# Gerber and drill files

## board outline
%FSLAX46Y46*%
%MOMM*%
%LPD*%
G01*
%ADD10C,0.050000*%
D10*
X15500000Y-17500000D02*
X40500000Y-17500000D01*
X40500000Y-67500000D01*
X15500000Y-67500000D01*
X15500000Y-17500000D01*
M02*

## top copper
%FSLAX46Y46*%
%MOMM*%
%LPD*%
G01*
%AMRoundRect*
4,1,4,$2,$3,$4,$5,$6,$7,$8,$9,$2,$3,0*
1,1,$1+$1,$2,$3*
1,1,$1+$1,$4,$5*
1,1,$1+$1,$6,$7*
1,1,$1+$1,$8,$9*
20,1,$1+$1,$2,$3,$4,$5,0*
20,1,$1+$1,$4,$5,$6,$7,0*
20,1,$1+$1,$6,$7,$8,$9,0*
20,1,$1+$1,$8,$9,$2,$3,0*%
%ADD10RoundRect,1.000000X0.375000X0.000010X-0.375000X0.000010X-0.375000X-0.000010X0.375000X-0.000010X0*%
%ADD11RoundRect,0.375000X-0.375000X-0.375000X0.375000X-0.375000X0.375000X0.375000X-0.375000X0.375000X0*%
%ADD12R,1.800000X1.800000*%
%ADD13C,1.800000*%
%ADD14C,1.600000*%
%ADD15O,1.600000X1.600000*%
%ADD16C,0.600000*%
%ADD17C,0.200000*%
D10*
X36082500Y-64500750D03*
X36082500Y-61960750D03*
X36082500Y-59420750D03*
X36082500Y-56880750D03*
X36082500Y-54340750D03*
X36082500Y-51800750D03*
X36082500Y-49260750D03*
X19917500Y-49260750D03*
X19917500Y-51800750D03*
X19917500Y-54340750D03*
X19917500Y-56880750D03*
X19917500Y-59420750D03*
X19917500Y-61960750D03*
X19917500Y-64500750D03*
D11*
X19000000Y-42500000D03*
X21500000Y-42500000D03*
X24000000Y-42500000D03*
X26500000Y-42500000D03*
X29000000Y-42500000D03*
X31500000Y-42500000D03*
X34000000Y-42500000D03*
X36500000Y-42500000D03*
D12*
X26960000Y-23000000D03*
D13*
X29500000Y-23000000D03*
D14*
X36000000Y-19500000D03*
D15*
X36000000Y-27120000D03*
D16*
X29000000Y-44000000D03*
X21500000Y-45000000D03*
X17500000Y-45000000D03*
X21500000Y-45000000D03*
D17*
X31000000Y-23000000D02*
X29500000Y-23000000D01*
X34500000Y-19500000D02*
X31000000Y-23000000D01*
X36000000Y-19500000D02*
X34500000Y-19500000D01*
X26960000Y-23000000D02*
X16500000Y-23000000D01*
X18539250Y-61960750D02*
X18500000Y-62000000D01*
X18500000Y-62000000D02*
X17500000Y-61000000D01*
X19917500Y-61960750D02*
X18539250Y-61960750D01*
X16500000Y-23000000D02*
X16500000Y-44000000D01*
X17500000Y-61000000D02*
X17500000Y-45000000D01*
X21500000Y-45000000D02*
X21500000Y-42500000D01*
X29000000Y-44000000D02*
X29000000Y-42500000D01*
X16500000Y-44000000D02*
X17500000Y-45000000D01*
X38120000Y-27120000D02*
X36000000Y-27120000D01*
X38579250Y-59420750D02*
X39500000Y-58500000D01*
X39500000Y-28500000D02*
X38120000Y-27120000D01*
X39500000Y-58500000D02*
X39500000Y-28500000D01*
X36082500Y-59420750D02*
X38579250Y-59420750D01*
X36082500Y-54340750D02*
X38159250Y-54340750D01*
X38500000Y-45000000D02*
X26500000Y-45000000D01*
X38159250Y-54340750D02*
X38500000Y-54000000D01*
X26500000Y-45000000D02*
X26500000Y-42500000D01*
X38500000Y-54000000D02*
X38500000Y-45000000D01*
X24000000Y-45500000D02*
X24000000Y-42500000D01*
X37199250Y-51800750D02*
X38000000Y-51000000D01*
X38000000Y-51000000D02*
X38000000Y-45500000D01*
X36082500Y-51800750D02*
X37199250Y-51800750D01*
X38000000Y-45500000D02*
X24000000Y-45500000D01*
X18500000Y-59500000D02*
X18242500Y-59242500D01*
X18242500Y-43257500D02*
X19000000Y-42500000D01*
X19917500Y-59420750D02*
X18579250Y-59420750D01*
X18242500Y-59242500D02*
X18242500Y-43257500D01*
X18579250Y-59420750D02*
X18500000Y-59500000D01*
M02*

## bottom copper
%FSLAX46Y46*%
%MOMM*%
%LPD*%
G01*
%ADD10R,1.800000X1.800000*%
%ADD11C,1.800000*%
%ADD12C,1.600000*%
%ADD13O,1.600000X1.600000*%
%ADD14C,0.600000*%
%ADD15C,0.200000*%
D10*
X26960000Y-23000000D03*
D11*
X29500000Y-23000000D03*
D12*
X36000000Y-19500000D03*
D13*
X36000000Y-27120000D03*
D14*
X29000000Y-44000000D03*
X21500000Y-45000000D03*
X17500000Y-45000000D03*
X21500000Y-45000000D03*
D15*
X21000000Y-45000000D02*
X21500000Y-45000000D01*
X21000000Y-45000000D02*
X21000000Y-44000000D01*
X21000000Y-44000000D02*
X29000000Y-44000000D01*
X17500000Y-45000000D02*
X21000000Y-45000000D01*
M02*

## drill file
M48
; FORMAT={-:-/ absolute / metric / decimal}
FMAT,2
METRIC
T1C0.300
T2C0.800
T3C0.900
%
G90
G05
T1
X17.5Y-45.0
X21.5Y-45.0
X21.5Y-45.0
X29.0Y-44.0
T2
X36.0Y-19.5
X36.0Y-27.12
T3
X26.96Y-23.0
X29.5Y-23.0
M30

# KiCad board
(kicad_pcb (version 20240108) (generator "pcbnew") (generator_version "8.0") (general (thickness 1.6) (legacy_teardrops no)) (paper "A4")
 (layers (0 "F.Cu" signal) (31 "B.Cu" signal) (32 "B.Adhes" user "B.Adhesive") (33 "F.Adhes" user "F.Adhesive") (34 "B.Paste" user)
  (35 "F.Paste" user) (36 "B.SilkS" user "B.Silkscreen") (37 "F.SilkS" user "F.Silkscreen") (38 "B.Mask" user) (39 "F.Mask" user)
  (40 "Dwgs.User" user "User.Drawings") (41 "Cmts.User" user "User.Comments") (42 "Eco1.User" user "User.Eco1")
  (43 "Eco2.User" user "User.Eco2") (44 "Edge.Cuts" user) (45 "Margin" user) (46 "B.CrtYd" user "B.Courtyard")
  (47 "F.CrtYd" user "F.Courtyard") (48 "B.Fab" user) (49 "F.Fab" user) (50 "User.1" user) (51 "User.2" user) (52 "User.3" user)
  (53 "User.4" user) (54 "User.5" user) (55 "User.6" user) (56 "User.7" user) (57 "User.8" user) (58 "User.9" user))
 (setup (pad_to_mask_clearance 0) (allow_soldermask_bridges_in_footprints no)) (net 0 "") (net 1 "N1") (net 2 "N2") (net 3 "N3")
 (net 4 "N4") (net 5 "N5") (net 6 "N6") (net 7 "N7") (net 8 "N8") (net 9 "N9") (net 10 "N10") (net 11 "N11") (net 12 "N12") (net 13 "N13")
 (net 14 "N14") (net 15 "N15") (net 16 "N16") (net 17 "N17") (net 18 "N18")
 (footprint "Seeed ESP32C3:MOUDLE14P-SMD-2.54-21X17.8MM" (layer "F.Cu") (at 36.9175 46.38075 180)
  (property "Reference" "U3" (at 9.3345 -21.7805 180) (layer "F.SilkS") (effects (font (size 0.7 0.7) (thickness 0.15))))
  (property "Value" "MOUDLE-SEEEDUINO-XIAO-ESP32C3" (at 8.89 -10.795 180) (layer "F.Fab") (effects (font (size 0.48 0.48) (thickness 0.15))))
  (pad "1" smd roundrect (at 0.835 -18.12 180) (size 2.75 2) (layers "F.Cu" "F.Paste" "F.Mask") (roundrect_rratio 0.5) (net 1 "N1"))
  (pad "2" smd roundrect (at 0.835 -15.58 180) (size 2.75 2) (layers "F.Cu" "F.Paste" "F.Mask") (roundrect_rratio 0.5) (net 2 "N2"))
  (pad "3" smd roundrect (at 0.835 -13.04 180) (size 2.75 2) (layers "F.Cu" "F.Paste" "F.Mask") (roundrect_rratio 0.5) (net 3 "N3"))
  (pad "4" smd roundrect (at 0.835 -10.5 180) (size 2.75 2) (layers "F.Cu" "F.Paste" "F.Mask") (roundrect_rratio 0.5) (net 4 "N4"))
  (pad "5" smd roundrect (at 0.835 -7.96 180) (size 2.75 2) (layers "F.Cu" "F.Paste" "F.Mask") (roundrect_rratio 0.5) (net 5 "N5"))
  (pad "6" smd roundrect (at 0.835 -5.42 180) (size 2.75 2) (layers "F.Cu" "F.Paste" "F.Mask") (roundrect_rratio 0.5) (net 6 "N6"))
  (pad "7" smd roundrect (at 0.835 -2.88 180) (size 2.75 2) (layers "F.Cu" "F.Paste" "F.Mask") (roundrect_rratio 0.5) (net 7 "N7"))
  (pad "8" smd roundrect (at 17 -2.88 180) (size 2.75 2) (layers "F.Cu" "F.Paste" "F.Mask") (roundrect_rratio 0.5) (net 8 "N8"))
  (pad "9" smd roundrect (at 17 -5.42 180) (size 2.75 2) (layers "F.Cu" "F.Paste" "F.Mask") (roundrect_rratio 0.5) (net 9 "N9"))
  (pad "10" smd roundrect (at 17 -7.96 180) (size 2.75 2) (layers "F.Cu" "F.Paste" "F.Mask") (roundrect_rratio 0.5) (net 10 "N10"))
  (pad "11" smd roundrect (at 17 -10.5 180) (size 2.75 2) (layers "F.Cu" "F.Paste" "F.Mask") (roundrect_rratio 0.5) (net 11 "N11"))
  (pad "12" smd roundrect (at 17 -13.04 180) (size 2.75 2) (layers "F.Cu" "F.Paste" "F.Mask") (roundrect_rratio 0.5) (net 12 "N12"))
  (pad "13" smd roundrect (at 17 -15.58 180) (size 2.75 2) (layers "F.Cu" "F.Paste" "F.Mask") (roundrect_rratio 0.5) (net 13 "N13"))
  (pad "14" smd roundrect (at 17 -18.12 180) (size 2.75 2) (layers "F.Cu" "F.Paste" "F.Mask") (roundrect_rratio 0.5) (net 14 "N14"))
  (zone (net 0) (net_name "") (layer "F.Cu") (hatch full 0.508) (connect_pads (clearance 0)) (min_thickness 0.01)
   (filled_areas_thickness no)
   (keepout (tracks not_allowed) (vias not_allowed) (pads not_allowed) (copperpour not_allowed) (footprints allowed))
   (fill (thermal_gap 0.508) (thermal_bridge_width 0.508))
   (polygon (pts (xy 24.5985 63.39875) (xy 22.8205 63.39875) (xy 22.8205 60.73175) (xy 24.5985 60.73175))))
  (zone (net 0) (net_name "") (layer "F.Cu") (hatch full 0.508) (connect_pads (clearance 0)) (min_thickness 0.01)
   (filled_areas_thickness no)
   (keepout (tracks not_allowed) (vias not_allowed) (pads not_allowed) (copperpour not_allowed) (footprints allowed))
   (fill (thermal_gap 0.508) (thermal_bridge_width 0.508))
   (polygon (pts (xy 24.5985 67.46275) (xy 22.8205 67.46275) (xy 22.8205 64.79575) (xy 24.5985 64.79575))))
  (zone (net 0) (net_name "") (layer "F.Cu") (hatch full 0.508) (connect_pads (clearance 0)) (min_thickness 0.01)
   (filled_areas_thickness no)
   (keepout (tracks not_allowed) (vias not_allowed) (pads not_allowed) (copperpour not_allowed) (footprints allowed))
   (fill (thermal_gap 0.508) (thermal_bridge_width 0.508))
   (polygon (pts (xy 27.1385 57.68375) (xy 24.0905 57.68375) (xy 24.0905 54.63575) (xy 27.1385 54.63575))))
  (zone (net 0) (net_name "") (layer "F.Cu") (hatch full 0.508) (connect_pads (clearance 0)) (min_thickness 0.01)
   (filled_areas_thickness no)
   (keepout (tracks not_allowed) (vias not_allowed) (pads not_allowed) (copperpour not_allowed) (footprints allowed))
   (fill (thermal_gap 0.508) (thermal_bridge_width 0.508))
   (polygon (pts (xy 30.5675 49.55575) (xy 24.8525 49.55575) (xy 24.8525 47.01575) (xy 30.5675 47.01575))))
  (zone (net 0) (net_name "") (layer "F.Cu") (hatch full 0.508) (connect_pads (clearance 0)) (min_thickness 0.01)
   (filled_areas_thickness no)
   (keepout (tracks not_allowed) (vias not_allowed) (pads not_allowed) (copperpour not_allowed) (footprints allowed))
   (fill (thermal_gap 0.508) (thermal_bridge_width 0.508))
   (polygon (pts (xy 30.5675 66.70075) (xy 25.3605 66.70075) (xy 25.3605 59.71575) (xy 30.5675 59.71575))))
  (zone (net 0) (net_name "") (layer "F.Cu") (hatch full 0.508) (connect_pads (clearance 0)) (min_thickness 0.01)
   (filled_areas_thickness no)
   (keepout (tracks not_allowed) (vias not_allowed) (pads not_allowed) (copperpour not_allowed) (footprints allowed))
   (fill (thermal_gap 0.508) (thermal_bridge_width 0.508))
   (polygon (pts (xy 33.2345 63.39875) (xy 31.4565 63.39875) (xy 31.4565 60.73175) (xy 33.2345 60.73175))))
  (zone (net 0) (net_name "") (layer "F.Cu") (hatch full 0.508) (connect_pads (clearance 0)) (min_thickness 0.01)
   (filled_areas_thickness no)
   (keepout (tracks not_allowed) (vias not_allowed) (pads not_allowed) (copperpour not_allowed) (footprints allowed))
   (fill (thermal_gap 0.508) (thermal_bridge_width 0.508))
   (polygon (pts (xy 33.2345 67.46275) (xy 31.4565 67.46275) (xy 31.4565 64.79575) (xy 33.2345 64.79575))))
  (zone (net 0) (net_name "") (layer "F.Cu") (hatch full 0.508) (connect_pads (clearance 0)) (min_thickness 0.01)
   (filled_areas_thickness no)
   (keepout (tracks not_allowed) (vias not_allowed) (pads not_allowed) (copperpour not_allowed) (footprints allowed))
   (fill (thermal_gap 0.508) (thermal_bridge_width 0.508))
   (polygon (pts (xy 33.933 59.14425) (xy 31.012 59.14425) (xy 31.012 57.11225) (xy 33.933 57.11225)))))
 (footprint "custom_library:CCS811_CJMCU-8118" (layer "F.Cu") (at 27.75 42.5)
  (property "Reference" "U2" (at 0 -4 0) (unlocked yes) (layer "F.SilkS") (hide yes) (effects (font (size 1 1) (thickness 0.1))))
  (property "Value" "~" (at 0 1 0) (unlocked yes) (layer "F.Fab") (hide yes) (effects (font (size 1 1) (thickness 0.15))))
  (pad "1" smd roundrect (at -8.75 0) (size 1.5 1.5) (layers "F.Cu" "F.Paste" "F.Mask") (roundrect_rratio 0.25) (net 12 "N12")
   (thermal_bridge_angle 45))
  (pad "2" smd roundrect (at -6.25 0) (size 1.5 1.5) (layers "F.Cu" "F.Paste" "F.Mask") (roundrect_rratio 0.25) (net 13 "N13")
   (thermal_bridge_angle 45))
  (pad "3" smd roundrect (at -3.75 0) (size 1.5 1.5) (layers "F.Cu" "F.Paste" "F.Mask") (roundrect_rratio 0.25) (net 6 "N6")
   (thermal_bridge_angle 45))
  (pad "4" smd roundrect (at -1.25 0) (size 1.5 1.5) (layers "F.Cu" "F.Paste" "F.Mask") (roundrect_rratio 0.25) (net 5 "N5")
   (thermal_bridge_angle 45))
  (pad "5" smd roundrect (at 1.25 0) (size 1.5 1.5) (layers "F.Cu" "F.Paste" "F.Mask") (roundrect_rratio 0.25) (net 13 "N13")
   (thermal_bridge_angle 45))
  (pad "6" smd roundrect (at 3.75 0) (size 1.5 1.5) (layers "F.Cu" "F.Paste" "F.Mask") (roundrect_rratio 0.25) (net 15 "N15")
   (thermal_bridge_angle 45))
  (pad "7" smd roundrect (at 6.25 0) (size 1.5 1.5) (layers "F.Cu" "F.Paste" "F.Mask") (roundrect_rratio 0.25) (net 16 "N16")
   (thermal_bridge_angle 45))
  (pad "8" smd roundrect (at 8.75 0) (size 1.5 1.5) (layers "F.Cu" "F.Paste" "F.Mask") (roundrect_rratio 0.25) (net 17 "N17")
   (thermal_bridge_angle 45)))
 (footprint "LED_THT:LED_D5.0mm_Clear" (layer "F.Cu") (at 26.96 23)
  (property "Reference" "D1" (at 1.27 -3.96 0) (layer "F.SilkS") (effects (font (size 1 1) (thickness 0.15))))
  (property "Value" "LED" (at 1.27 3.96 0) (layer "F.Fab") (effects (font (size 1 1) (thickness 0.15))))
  (pad "1" thru_hole rect (at 0 0) (size 1.8 1.8) (drill 0.9) (layers "*.Cu" "*.Mask") (remove_unused_layers no) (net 13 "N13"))
  (pad "2" thru_hole circle (at 2.54 0) (size 1.8 1.8) (drill 0.9) (layers "*.Cu" "*.Mask") (remove_unused_layers no) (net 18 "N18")))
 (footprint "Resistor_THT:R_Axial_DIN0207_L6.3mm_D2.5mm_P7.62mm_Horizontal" (layer "F.Cu") (at 36 19.5 -90)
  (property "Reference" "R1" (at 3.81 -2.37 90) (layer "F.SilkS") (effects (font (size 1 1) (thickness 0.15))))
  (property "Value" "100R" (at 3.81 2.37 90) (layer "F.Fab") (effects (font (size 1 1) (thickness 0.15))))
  (pad "1" thru_hole circle (at 0 0 270) (size 1.6 1.6) (drill 0.8) (layers "*.Cu" "*.Mask") (remove_unused_layers no) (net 18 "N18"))
  (pad "2" thru_hole oval (at 7.62 0 270) (size 1.6 1.6) (drill 0.8) (layers "*.Cu" "*.Mask") (remove_unused_layers no) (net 3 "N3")))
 (gr_rect (start 15.5 17.5) (end 40.5 67.5) (stroke (width 0.05) (type default)) (fill none) (layer "Edge.Cuts"))
 (segment (start 31 23) (end 29.5 23) (width 0.2) (layer "F.Cu") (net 18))
 (segment (start 34.5 19.5) (end 31 23) (width 0.2) (layer "F.Cu") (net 18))
 (segment (start 36 19.5) (end 34.5 19.5) (width 0.2) (layer "F.Cu") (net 18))
 (segment (start 26.96 23) (end 16.5 23) (width 0.2) (layer "F.Cu") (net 13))
 (segment (start 18.53925 61.96075) (end 18.5 62) (width 0.2) (layer "F.Cu") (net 13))
 (segment (start 18.5 62) (end 17.5 61) (width 0.2) (layer "F.Cu") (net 13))
 (segment (start 19.9175 61.96075) (end 18.53925 61.96075) (width 0.2) (layer "F.Cu") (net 13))
 (segment (start 16.5 23) (end 16.5 44) (width 0.2) (layer "F.Cu") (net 13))
 (segment (start 17.5 61) (end 17.5 45) (width 0.2) (layer "F.Cu") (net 13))
 (segment (start 21.5 45) (end 21.5 42.5) (width 0.2) (layer "F.Cu") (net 13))
 (segment (start 29 44) (end 29 42.5) (width 0.2) (layer "F.Cu") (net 13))
 (segment (start 16.5 44) (end 17.5 45) (width 0.2) (layer "F.Cu") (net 13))
 (via (at 29 44) (size 0.6) (drill 0.3) (layers "F.Cu" "B.Cu") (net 13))
 (via (at 21.5 45) (size 0.6) (drill 0.3) (layers "F.Cu" "B.Cu") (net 13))
 (via (at 17.5 45) (size 0.6) (drill 0.3) (layers "F.Cu" "B.Cu") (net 13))
 (via (at 21.5 45) (size 0.6) (drill 0.3) (layers "F.Cu" "B.Cu") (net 13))
 (segment (start 21 45) (end 21.5 45) (width 0.2) (layer "B.Cu") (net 13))
 (segment (start 21 45) (end 21 44) (width 0.2) (layer "B.Cu") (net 13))
 (segment (start 21 44) (end 29 44) (width 0.2) (layer "B.Cu") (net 13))
 (segment (start 17.5 45) (end 21 45) (width 0.2) (layer "B.Cu") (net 13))
 (segment (start 38.12 27.12) (end 36 27.12) (width 0.2) (layer "F.Cu") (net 3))
 (segment (start 38.57925 59.42075) (end 39.5 58.5) (width 0.2) (layer "F.Cu") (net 3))
 (segment (start 39.5 28.5) (end 38.12 27.12) (width 0.2) (layer "F.Cu") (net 3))
 (segment (start 39.5 58.5) (end 39.5 28.5) (width 0.2) (layer "F.Cu") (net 3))
 (segment (start 36.0825 59.42075) (end 38.57925 59.42075) (width 0.2) (layer "F.Cu") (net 3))
 (segment (start 36.0825 54.34075) (end 38.15925 54.34075) (width 0.2) (layer "F.Cu") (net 5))
 (segment (start 38.5 45) (end 26.5 45) (width 0.2) (layer "F.Cu") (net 5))
 (segment (start 38.15925 54.34075) (end 38.5 54) (width 0.2) (layer "F.Cu") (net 5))
 (segment (start 26.5 45) (end 26.5 42.5) (width 0.2) (layer "F.Cu") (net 5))
 (segment (start 38.5 54) (end 38.5 45) (width 0.2) (layer "F.Cu") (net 5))
 (segment (start 24 45.5) (end 24 42.5) (width 0.2) (layer "F.Cu") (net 6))
 (segment (start 37.19925 51.80075) (end 38 51) (width 0.2) (layer "F.Cu") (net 6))
 (segment (start 38 51) (end 38 45.5) (width 0.2) (layer "F.Cu") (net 6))
 (segment (start 36.0825 51.80075) (end 37.19925 51.80075) (width 0.2) (layer "F.Cu") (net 6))
 (segment (start 38 45.5) (end 24 45.5) (width 0.2) (layer "F.Cu") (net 6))
 (segment (start 18.5 59.5) (end 18.2425 59.2425) (width 0.2) (layer "F.Cu") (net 12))
 (segment (start 18.2425 43.2575) (end 19 42.5) (width 0.2) (layer "F.Cu") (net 12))
 (segment (start 19.9175 59.42075) (end 18.57925 59.42075) (width 0.2) (layer "F.Cu") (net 12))
 (segment (start 18.2425 59.2425) (end 18.2425 43.2575) (width 0.2) (layer "F.Cu") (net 12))
 (segment (start 18.57925 59.42075) (end 18.5 59.5) (width 0.2) (layer "F.Cu") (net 12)))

